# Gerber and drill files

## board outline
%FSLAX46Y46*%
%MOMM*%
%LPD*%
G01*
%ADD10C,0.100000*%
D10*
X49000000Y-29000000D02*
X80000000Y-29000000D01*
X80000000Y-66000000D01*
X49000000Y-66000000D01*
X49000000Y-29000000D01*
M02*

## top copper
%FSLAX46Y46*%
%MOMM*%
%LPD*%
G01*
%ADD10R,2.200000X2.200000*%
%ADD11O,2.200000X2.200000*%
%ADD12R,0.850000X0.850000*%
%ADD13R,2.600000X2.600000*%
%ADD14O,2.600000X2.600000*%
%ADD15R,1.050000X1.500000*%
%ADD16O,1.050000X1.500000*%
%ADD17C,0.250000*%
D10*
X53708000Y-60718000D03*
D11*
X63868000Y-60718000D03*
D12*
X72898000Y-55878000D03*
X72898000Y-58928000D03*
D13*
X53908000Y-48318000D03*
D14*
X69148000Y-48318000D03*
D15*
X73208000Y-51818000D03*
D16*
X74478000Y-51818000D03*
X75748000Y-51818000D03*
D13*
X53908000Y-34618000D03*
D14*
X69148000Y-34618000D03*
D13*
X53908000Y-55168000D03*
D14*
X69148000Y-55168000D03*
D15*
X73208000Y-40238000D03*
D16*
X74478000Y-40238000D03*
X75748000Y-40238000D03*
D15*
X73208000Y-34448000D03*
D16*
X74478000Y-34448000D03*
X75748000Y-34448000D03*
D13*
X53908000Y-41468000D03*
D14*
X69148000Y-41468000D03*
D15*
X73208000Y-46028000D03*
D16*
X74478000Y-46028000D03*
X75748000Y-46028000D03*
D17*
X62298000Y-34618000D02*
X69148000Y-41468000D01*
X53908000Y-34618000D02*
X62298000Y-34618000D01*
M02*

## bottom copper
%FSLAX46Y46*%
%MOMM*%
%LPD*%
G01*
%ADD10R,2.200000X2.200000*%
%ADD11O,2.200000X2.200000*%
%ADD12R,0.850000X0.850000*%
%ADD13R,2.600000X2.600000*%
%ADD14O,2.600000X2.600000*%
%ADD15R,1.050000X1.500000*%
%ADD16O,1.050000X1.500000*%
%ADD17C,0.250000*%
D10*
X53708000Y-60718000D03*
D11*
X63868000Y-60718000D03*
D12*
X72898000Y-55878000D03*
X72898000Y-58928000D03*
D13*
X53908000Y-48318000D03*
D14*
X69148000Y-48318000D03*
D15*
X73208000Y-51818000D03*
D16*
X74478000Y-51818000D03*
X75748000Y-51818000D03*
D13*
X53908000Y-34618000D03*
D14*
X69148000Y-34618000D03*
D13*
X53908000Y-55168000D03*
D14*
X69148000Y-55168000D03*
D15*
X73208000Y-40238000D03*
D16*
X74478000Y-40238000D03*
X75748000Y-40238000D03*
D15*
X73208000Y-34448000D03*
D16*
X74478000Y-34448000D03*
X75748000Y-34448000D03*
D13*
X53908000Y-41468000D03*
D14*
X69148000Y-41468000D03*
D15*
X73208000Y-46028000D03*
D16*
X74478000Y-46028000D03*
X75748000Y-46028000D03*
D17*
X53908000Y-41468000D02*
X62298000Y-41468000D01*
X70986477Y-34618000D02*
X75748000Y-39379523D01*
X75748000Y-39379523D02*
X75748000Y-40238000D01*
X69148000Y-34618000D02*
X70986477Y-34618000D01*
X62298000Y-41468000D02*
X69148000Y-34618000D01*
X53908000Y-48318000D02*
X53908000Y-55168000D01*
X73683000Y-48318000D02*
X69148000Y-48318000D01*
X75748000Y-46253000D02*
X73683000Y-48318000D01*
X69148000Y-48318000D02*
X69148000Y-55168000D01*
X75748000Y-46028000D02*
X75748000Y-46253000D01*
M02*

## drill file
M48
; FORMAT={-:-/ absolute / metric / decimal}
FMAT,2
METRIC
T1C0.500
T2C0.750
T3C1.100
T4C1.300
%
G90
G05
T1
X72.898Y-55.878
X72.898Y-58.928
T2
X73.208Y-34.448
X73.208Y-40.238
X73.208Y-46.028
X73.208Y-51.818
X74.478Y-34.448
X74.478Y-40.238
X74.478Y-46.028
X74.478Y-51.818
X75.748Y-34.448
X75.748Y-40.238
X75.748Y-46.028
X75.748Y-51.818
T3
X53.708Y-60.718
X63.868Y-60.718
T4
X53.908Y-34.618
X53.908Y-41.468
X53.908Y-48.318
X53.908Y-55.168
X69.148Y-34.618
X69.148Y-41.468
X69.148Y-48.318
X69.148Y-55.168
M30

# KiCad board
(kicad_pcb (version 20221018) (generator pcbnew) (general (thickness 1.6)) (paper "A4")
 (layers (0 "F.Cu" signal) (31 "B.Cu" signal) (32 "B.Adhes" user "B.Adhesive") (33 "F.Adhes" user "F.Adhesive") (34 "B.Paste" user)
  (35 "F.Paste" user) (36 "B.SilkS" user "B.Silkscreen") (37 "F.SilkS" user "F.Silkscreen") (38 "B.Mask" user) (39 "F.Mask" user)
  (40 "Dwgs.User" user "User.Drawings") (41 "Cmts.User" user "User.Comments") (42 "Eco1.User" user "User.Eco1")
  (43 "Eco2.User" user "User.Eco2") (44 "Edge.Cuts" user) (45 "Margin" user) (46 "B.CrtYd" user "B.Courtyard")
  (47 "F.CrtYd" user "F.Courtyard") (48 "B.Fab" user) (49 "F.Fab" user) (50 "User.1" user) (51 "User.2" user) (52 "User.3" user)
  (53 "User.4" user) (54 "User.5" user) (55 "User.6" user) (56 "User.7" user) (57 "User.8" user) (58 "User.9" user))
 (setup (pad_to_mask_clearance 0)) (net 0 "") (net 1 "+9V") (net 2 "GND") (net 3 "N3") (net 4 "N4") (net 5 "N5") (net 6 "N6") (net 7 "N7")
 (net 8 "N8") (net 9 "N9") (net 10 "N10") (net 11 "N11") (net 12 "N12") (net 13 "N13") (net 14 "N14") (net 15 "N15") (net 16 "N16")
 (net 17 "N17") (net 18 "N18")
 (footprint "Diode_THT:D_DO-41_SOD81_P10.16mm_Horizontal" (layer "F.Cu") (at 53.708 60.718)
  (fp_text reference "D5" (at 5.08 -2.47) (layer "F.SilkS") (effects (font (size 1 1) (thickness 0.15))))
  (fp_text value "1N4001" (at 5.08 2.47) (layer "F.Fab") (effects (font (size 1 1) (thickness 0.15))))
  (pad "1" thru_hole rect (at 0 0) (size 2.2 2.2) (drill 1.1) (layers "*.Cu" "*.Mask") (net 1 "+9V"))
  (pad "2" thru_hole oval (at 10.16 0) (size 2.2 2.2) (drill 1.1) (layers "*.Cu" "*.Mask") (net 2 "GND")))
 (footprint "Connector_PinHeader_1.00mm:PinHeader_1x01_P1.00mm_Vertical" (layer "F.Cu") (at 72.898 55.878)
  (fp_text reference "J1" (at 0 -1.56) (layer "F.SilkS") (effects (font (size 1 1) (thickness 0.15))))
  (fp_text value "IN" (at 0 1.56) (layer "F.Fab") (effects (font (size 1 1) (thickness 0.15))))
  (pad "1" thru_hole rect (at 0 0) (size 0.85 0.85) (drill 0.5) (layers "*.Cu" "*.Mask") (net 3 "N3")))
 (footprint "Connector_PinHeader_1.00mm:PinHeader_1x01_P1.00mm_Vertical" (layer "F.Cu") (at 72.898 58.928)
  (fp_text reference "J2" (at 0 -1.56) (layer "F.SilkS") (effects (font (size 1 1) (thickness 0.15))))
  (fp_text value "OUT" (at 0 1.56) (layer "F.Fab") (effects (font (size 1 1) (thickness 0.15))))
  (pad "1" thru_hole rect (at 0 0) (size 0.85 0.85) (drill 0.5) (layers "*.Cu" "*.Mask") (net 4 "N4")))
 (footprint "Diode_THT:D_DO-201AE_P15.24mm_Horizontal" (layer "F.Cu") (at 53.908 48.318)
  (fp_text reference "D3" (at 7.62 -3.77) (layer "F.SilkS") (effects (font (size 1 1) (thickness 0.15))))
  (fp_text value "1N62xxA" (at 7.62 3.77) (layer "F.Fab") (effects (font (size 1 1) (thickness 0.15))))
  (pad "1" thru_hole rect (at 0 0) (size 2.6 2.6) (drill 1.3) (layers "*.Cu" "*.Mask") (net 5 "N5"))
  (pad "2" thru_hole oval (at 15.24 0) (size 2.6 2.6) (drill 1.3) (layers "*.Cu" "*.Mask") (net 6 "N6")))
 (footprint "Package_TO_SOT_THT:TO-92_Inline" (layer "F.Cu") (at 73.208 51.818)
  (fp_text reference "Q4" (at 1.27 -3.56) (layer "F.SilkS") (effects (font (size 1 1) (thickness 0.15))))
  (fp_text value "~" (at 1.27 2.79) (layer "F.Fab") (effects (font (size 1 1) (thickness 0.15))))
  (pad "1" thru_hole rect (at 0 0) (size 1.05 1.5) (drill 0.75) (layers "*.Cu" "*.Mask") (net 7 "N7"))
  (pad "2" thru_hole oval (at 1.27 0) (size 1.05 1.5) (drill 0.75) (layers "*.Cu" "*.Mask") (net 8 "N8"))
  (pad "3" thru_hole oval (at 2.54 0) (size 1.05 1.5) (drill 0.75) (layers "*.Cu" "*.Mask") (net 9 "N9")))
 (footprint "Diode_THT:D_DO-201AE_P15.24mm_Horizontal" (layer "F.Cu") (at 53.908 34.618)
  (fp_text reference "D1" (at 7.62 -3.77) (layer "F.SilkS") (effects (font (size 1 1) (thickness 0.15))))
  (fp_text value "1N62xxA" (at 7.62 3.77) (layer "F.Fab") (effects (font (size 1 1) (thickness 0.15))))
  (pad "1" thru_hole rect (at 0 0) (size 2.6 2.6) (drill 1.3) (layers "*.Cu" "*.Mask") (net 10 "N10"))
  (pad "2" thru_hole oval (at 15.24 0) (size 2.6 2.6) (drill 1.3) (layers "*.Cu" "*.Mask") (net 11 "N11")))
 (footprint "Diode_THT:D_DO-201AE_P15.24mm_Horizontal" (layer "F.Cu") (at 53.908 55.168)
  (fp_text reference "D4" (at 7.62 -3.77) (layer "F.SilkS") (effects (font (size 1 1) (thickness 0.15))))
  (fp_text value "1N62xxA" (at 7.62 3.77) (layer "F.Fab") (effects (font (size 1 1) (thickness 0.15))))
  (pad "1" thru_hole rect (at 0 0) (size 2.6 2.6) (drill 1.3) (layers "*.Cu" "*.Mask") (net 5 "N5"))
  (pad "2" thru_hole oval (at 15.24 0) (size 2.6 2.6) (drill 1.3) (layers "*.Cu" "*.Mask") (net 6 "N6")))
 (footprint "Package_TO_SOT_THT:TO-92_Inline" (layer "F.Cu") (at 73.208 40.238)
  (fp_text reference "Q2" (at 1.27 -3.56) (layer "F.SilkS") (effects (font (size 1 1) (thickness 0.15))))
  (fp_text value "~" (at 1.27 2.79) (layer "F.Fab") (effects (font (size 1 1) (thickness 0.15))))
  (pad "1" thru_hole rect (at 0 0) (size 1.05 1.5) (drill 0.75) (layers "*.Cu" "*.Mask") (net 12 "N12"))
  (pad "2" thru_hole oval (at 1.27 0) (size 1.05 1.5) (drill 0.75) (layers "*.Cu" "*.Mask") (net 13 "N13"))
  (pad "3" thru_hole oval (at 2.54 0) (size 1.05 1.5) (drill 0.75) (layers "*.Cu" "*.Mask") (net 11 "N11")))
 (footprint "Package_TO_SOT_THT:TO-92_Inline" (layer "F.Cu") (at 73.208 34.448)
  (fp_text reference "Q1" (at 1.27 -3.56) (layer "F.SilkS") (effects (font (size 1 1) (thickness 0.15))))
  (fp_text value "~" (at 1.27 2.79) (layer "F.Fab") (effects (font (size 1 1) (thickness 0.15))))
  (pad "1" thru_hole rect (at 0 0) (size 1.05 1.5) (drill 0.75) (layers "*.Cu" "*.Mask") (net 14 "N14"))
  (pad "2" thru_hole oval (at 1.27 0) (size 1.05 1.5) (drill 0.75) (layers "*.Cu" "*.Mask") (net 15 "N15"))
  (pad "3" thru_hole oval (at 2.54 0) (size 1.05 1.5) (drill 0.75) (layers "*.Cu" "*.Mask") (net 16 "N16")))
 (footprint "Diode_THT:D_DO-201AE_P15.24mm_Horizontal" (layer "F.Cu") (at 53.908 41.468)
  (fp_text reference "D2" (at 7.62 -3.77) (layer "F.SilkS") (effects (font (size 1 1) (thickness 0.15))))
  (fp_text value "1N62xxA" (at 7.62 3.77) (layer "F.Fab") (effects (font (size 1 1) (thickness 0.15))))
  (pad "1" thru_hole rect (at 0 0) (size 2.6 2.6) (drill 1.3) (layers "*.Cu" "*.Mask") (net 11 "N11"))
  (pad "2" thru_hole oval (at 15.24 0) (size 2.6 2.6) (drill 1.3) (layers "*.Cu" "*.Mask") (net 10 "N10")))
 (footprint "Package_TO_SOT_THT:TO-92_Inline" (layer "F.Cu") (at 73.208 46.028)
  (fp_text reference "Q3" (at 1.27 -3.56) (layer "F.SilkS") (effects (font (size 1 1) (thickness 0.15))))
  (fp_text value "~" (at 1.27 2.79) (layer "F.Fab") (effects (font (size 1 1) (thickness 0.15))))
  (pad "1" thru_hole rect (at 0 0) (size 1.05 1.5) (drill 0.75) (layers "*.Cu" "*.Mask") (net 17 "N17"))
  (pad "2" thru_hole oval (at 1.27 0) (size 1.05 1.5) (drill 0.75) (layers "*.Cu" "*.Mask") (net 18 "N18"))
  (pad "3" thru_hole oval (at 2.54 0) (size 1.05 1.5) (drill 0.75) (layers "*.Cu" "*.Mask") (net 6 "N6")))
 (gr_rect (start 49 29) (end 80 66) (stroke (width 0.1) (type default)) (fill none) (layer "Edge.Cuts"))
 (segment (start 62.298 34.618) (end 69.148 41.468) (width 0.25) (layer "F.Cu") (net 10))
 (segment (start 53.908 34.618) (end 62.298 34.618) (width 0.25) (layer "F.Cu") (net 10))
 (segment (start 53.908 41.468) (end 62.298 41.468) (width 0.25) (layer "B.Cu") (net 11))
 (segment (start 70.986477 34.618) (end 75.748 39.379523) (width 0.25) (layer "B.Cu") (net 11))
 (segment (start 75.748 39.379523) (end 75.748 40.238) (width 0.25) (layer "B.Cu") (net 11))
 (segment (start 69.148 34.618) (end 70.986477 34.618) (width 0.25) (layer "B.Cu") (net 11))
 (segment (start 62.298 41.468) (end 69.148 34.618) (width 0.25) (layer "B.Cu") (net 11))
 (segment (start 53.908 48.318) (end 53.908 55.168) (width 0.25) (layer "B.Cu") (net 5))
 (segment (start 73.683 48.318) (end 69.148 48.318) (width 0.25) (layer "B.Cu") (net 6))
 (segment (start 75.748 46.253) (end 73.683 48.318) (width 0.25) (layer "B.Cu") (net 6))
 (segment (start 69.148 48.318) (end 69.148 55.168) (width 0.25) (layer "B.Cu") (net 6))
 (segment (start 75.748 46.028) (end 75.748 46.253) (width 0.25) (layer "B.Cu") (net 6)))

